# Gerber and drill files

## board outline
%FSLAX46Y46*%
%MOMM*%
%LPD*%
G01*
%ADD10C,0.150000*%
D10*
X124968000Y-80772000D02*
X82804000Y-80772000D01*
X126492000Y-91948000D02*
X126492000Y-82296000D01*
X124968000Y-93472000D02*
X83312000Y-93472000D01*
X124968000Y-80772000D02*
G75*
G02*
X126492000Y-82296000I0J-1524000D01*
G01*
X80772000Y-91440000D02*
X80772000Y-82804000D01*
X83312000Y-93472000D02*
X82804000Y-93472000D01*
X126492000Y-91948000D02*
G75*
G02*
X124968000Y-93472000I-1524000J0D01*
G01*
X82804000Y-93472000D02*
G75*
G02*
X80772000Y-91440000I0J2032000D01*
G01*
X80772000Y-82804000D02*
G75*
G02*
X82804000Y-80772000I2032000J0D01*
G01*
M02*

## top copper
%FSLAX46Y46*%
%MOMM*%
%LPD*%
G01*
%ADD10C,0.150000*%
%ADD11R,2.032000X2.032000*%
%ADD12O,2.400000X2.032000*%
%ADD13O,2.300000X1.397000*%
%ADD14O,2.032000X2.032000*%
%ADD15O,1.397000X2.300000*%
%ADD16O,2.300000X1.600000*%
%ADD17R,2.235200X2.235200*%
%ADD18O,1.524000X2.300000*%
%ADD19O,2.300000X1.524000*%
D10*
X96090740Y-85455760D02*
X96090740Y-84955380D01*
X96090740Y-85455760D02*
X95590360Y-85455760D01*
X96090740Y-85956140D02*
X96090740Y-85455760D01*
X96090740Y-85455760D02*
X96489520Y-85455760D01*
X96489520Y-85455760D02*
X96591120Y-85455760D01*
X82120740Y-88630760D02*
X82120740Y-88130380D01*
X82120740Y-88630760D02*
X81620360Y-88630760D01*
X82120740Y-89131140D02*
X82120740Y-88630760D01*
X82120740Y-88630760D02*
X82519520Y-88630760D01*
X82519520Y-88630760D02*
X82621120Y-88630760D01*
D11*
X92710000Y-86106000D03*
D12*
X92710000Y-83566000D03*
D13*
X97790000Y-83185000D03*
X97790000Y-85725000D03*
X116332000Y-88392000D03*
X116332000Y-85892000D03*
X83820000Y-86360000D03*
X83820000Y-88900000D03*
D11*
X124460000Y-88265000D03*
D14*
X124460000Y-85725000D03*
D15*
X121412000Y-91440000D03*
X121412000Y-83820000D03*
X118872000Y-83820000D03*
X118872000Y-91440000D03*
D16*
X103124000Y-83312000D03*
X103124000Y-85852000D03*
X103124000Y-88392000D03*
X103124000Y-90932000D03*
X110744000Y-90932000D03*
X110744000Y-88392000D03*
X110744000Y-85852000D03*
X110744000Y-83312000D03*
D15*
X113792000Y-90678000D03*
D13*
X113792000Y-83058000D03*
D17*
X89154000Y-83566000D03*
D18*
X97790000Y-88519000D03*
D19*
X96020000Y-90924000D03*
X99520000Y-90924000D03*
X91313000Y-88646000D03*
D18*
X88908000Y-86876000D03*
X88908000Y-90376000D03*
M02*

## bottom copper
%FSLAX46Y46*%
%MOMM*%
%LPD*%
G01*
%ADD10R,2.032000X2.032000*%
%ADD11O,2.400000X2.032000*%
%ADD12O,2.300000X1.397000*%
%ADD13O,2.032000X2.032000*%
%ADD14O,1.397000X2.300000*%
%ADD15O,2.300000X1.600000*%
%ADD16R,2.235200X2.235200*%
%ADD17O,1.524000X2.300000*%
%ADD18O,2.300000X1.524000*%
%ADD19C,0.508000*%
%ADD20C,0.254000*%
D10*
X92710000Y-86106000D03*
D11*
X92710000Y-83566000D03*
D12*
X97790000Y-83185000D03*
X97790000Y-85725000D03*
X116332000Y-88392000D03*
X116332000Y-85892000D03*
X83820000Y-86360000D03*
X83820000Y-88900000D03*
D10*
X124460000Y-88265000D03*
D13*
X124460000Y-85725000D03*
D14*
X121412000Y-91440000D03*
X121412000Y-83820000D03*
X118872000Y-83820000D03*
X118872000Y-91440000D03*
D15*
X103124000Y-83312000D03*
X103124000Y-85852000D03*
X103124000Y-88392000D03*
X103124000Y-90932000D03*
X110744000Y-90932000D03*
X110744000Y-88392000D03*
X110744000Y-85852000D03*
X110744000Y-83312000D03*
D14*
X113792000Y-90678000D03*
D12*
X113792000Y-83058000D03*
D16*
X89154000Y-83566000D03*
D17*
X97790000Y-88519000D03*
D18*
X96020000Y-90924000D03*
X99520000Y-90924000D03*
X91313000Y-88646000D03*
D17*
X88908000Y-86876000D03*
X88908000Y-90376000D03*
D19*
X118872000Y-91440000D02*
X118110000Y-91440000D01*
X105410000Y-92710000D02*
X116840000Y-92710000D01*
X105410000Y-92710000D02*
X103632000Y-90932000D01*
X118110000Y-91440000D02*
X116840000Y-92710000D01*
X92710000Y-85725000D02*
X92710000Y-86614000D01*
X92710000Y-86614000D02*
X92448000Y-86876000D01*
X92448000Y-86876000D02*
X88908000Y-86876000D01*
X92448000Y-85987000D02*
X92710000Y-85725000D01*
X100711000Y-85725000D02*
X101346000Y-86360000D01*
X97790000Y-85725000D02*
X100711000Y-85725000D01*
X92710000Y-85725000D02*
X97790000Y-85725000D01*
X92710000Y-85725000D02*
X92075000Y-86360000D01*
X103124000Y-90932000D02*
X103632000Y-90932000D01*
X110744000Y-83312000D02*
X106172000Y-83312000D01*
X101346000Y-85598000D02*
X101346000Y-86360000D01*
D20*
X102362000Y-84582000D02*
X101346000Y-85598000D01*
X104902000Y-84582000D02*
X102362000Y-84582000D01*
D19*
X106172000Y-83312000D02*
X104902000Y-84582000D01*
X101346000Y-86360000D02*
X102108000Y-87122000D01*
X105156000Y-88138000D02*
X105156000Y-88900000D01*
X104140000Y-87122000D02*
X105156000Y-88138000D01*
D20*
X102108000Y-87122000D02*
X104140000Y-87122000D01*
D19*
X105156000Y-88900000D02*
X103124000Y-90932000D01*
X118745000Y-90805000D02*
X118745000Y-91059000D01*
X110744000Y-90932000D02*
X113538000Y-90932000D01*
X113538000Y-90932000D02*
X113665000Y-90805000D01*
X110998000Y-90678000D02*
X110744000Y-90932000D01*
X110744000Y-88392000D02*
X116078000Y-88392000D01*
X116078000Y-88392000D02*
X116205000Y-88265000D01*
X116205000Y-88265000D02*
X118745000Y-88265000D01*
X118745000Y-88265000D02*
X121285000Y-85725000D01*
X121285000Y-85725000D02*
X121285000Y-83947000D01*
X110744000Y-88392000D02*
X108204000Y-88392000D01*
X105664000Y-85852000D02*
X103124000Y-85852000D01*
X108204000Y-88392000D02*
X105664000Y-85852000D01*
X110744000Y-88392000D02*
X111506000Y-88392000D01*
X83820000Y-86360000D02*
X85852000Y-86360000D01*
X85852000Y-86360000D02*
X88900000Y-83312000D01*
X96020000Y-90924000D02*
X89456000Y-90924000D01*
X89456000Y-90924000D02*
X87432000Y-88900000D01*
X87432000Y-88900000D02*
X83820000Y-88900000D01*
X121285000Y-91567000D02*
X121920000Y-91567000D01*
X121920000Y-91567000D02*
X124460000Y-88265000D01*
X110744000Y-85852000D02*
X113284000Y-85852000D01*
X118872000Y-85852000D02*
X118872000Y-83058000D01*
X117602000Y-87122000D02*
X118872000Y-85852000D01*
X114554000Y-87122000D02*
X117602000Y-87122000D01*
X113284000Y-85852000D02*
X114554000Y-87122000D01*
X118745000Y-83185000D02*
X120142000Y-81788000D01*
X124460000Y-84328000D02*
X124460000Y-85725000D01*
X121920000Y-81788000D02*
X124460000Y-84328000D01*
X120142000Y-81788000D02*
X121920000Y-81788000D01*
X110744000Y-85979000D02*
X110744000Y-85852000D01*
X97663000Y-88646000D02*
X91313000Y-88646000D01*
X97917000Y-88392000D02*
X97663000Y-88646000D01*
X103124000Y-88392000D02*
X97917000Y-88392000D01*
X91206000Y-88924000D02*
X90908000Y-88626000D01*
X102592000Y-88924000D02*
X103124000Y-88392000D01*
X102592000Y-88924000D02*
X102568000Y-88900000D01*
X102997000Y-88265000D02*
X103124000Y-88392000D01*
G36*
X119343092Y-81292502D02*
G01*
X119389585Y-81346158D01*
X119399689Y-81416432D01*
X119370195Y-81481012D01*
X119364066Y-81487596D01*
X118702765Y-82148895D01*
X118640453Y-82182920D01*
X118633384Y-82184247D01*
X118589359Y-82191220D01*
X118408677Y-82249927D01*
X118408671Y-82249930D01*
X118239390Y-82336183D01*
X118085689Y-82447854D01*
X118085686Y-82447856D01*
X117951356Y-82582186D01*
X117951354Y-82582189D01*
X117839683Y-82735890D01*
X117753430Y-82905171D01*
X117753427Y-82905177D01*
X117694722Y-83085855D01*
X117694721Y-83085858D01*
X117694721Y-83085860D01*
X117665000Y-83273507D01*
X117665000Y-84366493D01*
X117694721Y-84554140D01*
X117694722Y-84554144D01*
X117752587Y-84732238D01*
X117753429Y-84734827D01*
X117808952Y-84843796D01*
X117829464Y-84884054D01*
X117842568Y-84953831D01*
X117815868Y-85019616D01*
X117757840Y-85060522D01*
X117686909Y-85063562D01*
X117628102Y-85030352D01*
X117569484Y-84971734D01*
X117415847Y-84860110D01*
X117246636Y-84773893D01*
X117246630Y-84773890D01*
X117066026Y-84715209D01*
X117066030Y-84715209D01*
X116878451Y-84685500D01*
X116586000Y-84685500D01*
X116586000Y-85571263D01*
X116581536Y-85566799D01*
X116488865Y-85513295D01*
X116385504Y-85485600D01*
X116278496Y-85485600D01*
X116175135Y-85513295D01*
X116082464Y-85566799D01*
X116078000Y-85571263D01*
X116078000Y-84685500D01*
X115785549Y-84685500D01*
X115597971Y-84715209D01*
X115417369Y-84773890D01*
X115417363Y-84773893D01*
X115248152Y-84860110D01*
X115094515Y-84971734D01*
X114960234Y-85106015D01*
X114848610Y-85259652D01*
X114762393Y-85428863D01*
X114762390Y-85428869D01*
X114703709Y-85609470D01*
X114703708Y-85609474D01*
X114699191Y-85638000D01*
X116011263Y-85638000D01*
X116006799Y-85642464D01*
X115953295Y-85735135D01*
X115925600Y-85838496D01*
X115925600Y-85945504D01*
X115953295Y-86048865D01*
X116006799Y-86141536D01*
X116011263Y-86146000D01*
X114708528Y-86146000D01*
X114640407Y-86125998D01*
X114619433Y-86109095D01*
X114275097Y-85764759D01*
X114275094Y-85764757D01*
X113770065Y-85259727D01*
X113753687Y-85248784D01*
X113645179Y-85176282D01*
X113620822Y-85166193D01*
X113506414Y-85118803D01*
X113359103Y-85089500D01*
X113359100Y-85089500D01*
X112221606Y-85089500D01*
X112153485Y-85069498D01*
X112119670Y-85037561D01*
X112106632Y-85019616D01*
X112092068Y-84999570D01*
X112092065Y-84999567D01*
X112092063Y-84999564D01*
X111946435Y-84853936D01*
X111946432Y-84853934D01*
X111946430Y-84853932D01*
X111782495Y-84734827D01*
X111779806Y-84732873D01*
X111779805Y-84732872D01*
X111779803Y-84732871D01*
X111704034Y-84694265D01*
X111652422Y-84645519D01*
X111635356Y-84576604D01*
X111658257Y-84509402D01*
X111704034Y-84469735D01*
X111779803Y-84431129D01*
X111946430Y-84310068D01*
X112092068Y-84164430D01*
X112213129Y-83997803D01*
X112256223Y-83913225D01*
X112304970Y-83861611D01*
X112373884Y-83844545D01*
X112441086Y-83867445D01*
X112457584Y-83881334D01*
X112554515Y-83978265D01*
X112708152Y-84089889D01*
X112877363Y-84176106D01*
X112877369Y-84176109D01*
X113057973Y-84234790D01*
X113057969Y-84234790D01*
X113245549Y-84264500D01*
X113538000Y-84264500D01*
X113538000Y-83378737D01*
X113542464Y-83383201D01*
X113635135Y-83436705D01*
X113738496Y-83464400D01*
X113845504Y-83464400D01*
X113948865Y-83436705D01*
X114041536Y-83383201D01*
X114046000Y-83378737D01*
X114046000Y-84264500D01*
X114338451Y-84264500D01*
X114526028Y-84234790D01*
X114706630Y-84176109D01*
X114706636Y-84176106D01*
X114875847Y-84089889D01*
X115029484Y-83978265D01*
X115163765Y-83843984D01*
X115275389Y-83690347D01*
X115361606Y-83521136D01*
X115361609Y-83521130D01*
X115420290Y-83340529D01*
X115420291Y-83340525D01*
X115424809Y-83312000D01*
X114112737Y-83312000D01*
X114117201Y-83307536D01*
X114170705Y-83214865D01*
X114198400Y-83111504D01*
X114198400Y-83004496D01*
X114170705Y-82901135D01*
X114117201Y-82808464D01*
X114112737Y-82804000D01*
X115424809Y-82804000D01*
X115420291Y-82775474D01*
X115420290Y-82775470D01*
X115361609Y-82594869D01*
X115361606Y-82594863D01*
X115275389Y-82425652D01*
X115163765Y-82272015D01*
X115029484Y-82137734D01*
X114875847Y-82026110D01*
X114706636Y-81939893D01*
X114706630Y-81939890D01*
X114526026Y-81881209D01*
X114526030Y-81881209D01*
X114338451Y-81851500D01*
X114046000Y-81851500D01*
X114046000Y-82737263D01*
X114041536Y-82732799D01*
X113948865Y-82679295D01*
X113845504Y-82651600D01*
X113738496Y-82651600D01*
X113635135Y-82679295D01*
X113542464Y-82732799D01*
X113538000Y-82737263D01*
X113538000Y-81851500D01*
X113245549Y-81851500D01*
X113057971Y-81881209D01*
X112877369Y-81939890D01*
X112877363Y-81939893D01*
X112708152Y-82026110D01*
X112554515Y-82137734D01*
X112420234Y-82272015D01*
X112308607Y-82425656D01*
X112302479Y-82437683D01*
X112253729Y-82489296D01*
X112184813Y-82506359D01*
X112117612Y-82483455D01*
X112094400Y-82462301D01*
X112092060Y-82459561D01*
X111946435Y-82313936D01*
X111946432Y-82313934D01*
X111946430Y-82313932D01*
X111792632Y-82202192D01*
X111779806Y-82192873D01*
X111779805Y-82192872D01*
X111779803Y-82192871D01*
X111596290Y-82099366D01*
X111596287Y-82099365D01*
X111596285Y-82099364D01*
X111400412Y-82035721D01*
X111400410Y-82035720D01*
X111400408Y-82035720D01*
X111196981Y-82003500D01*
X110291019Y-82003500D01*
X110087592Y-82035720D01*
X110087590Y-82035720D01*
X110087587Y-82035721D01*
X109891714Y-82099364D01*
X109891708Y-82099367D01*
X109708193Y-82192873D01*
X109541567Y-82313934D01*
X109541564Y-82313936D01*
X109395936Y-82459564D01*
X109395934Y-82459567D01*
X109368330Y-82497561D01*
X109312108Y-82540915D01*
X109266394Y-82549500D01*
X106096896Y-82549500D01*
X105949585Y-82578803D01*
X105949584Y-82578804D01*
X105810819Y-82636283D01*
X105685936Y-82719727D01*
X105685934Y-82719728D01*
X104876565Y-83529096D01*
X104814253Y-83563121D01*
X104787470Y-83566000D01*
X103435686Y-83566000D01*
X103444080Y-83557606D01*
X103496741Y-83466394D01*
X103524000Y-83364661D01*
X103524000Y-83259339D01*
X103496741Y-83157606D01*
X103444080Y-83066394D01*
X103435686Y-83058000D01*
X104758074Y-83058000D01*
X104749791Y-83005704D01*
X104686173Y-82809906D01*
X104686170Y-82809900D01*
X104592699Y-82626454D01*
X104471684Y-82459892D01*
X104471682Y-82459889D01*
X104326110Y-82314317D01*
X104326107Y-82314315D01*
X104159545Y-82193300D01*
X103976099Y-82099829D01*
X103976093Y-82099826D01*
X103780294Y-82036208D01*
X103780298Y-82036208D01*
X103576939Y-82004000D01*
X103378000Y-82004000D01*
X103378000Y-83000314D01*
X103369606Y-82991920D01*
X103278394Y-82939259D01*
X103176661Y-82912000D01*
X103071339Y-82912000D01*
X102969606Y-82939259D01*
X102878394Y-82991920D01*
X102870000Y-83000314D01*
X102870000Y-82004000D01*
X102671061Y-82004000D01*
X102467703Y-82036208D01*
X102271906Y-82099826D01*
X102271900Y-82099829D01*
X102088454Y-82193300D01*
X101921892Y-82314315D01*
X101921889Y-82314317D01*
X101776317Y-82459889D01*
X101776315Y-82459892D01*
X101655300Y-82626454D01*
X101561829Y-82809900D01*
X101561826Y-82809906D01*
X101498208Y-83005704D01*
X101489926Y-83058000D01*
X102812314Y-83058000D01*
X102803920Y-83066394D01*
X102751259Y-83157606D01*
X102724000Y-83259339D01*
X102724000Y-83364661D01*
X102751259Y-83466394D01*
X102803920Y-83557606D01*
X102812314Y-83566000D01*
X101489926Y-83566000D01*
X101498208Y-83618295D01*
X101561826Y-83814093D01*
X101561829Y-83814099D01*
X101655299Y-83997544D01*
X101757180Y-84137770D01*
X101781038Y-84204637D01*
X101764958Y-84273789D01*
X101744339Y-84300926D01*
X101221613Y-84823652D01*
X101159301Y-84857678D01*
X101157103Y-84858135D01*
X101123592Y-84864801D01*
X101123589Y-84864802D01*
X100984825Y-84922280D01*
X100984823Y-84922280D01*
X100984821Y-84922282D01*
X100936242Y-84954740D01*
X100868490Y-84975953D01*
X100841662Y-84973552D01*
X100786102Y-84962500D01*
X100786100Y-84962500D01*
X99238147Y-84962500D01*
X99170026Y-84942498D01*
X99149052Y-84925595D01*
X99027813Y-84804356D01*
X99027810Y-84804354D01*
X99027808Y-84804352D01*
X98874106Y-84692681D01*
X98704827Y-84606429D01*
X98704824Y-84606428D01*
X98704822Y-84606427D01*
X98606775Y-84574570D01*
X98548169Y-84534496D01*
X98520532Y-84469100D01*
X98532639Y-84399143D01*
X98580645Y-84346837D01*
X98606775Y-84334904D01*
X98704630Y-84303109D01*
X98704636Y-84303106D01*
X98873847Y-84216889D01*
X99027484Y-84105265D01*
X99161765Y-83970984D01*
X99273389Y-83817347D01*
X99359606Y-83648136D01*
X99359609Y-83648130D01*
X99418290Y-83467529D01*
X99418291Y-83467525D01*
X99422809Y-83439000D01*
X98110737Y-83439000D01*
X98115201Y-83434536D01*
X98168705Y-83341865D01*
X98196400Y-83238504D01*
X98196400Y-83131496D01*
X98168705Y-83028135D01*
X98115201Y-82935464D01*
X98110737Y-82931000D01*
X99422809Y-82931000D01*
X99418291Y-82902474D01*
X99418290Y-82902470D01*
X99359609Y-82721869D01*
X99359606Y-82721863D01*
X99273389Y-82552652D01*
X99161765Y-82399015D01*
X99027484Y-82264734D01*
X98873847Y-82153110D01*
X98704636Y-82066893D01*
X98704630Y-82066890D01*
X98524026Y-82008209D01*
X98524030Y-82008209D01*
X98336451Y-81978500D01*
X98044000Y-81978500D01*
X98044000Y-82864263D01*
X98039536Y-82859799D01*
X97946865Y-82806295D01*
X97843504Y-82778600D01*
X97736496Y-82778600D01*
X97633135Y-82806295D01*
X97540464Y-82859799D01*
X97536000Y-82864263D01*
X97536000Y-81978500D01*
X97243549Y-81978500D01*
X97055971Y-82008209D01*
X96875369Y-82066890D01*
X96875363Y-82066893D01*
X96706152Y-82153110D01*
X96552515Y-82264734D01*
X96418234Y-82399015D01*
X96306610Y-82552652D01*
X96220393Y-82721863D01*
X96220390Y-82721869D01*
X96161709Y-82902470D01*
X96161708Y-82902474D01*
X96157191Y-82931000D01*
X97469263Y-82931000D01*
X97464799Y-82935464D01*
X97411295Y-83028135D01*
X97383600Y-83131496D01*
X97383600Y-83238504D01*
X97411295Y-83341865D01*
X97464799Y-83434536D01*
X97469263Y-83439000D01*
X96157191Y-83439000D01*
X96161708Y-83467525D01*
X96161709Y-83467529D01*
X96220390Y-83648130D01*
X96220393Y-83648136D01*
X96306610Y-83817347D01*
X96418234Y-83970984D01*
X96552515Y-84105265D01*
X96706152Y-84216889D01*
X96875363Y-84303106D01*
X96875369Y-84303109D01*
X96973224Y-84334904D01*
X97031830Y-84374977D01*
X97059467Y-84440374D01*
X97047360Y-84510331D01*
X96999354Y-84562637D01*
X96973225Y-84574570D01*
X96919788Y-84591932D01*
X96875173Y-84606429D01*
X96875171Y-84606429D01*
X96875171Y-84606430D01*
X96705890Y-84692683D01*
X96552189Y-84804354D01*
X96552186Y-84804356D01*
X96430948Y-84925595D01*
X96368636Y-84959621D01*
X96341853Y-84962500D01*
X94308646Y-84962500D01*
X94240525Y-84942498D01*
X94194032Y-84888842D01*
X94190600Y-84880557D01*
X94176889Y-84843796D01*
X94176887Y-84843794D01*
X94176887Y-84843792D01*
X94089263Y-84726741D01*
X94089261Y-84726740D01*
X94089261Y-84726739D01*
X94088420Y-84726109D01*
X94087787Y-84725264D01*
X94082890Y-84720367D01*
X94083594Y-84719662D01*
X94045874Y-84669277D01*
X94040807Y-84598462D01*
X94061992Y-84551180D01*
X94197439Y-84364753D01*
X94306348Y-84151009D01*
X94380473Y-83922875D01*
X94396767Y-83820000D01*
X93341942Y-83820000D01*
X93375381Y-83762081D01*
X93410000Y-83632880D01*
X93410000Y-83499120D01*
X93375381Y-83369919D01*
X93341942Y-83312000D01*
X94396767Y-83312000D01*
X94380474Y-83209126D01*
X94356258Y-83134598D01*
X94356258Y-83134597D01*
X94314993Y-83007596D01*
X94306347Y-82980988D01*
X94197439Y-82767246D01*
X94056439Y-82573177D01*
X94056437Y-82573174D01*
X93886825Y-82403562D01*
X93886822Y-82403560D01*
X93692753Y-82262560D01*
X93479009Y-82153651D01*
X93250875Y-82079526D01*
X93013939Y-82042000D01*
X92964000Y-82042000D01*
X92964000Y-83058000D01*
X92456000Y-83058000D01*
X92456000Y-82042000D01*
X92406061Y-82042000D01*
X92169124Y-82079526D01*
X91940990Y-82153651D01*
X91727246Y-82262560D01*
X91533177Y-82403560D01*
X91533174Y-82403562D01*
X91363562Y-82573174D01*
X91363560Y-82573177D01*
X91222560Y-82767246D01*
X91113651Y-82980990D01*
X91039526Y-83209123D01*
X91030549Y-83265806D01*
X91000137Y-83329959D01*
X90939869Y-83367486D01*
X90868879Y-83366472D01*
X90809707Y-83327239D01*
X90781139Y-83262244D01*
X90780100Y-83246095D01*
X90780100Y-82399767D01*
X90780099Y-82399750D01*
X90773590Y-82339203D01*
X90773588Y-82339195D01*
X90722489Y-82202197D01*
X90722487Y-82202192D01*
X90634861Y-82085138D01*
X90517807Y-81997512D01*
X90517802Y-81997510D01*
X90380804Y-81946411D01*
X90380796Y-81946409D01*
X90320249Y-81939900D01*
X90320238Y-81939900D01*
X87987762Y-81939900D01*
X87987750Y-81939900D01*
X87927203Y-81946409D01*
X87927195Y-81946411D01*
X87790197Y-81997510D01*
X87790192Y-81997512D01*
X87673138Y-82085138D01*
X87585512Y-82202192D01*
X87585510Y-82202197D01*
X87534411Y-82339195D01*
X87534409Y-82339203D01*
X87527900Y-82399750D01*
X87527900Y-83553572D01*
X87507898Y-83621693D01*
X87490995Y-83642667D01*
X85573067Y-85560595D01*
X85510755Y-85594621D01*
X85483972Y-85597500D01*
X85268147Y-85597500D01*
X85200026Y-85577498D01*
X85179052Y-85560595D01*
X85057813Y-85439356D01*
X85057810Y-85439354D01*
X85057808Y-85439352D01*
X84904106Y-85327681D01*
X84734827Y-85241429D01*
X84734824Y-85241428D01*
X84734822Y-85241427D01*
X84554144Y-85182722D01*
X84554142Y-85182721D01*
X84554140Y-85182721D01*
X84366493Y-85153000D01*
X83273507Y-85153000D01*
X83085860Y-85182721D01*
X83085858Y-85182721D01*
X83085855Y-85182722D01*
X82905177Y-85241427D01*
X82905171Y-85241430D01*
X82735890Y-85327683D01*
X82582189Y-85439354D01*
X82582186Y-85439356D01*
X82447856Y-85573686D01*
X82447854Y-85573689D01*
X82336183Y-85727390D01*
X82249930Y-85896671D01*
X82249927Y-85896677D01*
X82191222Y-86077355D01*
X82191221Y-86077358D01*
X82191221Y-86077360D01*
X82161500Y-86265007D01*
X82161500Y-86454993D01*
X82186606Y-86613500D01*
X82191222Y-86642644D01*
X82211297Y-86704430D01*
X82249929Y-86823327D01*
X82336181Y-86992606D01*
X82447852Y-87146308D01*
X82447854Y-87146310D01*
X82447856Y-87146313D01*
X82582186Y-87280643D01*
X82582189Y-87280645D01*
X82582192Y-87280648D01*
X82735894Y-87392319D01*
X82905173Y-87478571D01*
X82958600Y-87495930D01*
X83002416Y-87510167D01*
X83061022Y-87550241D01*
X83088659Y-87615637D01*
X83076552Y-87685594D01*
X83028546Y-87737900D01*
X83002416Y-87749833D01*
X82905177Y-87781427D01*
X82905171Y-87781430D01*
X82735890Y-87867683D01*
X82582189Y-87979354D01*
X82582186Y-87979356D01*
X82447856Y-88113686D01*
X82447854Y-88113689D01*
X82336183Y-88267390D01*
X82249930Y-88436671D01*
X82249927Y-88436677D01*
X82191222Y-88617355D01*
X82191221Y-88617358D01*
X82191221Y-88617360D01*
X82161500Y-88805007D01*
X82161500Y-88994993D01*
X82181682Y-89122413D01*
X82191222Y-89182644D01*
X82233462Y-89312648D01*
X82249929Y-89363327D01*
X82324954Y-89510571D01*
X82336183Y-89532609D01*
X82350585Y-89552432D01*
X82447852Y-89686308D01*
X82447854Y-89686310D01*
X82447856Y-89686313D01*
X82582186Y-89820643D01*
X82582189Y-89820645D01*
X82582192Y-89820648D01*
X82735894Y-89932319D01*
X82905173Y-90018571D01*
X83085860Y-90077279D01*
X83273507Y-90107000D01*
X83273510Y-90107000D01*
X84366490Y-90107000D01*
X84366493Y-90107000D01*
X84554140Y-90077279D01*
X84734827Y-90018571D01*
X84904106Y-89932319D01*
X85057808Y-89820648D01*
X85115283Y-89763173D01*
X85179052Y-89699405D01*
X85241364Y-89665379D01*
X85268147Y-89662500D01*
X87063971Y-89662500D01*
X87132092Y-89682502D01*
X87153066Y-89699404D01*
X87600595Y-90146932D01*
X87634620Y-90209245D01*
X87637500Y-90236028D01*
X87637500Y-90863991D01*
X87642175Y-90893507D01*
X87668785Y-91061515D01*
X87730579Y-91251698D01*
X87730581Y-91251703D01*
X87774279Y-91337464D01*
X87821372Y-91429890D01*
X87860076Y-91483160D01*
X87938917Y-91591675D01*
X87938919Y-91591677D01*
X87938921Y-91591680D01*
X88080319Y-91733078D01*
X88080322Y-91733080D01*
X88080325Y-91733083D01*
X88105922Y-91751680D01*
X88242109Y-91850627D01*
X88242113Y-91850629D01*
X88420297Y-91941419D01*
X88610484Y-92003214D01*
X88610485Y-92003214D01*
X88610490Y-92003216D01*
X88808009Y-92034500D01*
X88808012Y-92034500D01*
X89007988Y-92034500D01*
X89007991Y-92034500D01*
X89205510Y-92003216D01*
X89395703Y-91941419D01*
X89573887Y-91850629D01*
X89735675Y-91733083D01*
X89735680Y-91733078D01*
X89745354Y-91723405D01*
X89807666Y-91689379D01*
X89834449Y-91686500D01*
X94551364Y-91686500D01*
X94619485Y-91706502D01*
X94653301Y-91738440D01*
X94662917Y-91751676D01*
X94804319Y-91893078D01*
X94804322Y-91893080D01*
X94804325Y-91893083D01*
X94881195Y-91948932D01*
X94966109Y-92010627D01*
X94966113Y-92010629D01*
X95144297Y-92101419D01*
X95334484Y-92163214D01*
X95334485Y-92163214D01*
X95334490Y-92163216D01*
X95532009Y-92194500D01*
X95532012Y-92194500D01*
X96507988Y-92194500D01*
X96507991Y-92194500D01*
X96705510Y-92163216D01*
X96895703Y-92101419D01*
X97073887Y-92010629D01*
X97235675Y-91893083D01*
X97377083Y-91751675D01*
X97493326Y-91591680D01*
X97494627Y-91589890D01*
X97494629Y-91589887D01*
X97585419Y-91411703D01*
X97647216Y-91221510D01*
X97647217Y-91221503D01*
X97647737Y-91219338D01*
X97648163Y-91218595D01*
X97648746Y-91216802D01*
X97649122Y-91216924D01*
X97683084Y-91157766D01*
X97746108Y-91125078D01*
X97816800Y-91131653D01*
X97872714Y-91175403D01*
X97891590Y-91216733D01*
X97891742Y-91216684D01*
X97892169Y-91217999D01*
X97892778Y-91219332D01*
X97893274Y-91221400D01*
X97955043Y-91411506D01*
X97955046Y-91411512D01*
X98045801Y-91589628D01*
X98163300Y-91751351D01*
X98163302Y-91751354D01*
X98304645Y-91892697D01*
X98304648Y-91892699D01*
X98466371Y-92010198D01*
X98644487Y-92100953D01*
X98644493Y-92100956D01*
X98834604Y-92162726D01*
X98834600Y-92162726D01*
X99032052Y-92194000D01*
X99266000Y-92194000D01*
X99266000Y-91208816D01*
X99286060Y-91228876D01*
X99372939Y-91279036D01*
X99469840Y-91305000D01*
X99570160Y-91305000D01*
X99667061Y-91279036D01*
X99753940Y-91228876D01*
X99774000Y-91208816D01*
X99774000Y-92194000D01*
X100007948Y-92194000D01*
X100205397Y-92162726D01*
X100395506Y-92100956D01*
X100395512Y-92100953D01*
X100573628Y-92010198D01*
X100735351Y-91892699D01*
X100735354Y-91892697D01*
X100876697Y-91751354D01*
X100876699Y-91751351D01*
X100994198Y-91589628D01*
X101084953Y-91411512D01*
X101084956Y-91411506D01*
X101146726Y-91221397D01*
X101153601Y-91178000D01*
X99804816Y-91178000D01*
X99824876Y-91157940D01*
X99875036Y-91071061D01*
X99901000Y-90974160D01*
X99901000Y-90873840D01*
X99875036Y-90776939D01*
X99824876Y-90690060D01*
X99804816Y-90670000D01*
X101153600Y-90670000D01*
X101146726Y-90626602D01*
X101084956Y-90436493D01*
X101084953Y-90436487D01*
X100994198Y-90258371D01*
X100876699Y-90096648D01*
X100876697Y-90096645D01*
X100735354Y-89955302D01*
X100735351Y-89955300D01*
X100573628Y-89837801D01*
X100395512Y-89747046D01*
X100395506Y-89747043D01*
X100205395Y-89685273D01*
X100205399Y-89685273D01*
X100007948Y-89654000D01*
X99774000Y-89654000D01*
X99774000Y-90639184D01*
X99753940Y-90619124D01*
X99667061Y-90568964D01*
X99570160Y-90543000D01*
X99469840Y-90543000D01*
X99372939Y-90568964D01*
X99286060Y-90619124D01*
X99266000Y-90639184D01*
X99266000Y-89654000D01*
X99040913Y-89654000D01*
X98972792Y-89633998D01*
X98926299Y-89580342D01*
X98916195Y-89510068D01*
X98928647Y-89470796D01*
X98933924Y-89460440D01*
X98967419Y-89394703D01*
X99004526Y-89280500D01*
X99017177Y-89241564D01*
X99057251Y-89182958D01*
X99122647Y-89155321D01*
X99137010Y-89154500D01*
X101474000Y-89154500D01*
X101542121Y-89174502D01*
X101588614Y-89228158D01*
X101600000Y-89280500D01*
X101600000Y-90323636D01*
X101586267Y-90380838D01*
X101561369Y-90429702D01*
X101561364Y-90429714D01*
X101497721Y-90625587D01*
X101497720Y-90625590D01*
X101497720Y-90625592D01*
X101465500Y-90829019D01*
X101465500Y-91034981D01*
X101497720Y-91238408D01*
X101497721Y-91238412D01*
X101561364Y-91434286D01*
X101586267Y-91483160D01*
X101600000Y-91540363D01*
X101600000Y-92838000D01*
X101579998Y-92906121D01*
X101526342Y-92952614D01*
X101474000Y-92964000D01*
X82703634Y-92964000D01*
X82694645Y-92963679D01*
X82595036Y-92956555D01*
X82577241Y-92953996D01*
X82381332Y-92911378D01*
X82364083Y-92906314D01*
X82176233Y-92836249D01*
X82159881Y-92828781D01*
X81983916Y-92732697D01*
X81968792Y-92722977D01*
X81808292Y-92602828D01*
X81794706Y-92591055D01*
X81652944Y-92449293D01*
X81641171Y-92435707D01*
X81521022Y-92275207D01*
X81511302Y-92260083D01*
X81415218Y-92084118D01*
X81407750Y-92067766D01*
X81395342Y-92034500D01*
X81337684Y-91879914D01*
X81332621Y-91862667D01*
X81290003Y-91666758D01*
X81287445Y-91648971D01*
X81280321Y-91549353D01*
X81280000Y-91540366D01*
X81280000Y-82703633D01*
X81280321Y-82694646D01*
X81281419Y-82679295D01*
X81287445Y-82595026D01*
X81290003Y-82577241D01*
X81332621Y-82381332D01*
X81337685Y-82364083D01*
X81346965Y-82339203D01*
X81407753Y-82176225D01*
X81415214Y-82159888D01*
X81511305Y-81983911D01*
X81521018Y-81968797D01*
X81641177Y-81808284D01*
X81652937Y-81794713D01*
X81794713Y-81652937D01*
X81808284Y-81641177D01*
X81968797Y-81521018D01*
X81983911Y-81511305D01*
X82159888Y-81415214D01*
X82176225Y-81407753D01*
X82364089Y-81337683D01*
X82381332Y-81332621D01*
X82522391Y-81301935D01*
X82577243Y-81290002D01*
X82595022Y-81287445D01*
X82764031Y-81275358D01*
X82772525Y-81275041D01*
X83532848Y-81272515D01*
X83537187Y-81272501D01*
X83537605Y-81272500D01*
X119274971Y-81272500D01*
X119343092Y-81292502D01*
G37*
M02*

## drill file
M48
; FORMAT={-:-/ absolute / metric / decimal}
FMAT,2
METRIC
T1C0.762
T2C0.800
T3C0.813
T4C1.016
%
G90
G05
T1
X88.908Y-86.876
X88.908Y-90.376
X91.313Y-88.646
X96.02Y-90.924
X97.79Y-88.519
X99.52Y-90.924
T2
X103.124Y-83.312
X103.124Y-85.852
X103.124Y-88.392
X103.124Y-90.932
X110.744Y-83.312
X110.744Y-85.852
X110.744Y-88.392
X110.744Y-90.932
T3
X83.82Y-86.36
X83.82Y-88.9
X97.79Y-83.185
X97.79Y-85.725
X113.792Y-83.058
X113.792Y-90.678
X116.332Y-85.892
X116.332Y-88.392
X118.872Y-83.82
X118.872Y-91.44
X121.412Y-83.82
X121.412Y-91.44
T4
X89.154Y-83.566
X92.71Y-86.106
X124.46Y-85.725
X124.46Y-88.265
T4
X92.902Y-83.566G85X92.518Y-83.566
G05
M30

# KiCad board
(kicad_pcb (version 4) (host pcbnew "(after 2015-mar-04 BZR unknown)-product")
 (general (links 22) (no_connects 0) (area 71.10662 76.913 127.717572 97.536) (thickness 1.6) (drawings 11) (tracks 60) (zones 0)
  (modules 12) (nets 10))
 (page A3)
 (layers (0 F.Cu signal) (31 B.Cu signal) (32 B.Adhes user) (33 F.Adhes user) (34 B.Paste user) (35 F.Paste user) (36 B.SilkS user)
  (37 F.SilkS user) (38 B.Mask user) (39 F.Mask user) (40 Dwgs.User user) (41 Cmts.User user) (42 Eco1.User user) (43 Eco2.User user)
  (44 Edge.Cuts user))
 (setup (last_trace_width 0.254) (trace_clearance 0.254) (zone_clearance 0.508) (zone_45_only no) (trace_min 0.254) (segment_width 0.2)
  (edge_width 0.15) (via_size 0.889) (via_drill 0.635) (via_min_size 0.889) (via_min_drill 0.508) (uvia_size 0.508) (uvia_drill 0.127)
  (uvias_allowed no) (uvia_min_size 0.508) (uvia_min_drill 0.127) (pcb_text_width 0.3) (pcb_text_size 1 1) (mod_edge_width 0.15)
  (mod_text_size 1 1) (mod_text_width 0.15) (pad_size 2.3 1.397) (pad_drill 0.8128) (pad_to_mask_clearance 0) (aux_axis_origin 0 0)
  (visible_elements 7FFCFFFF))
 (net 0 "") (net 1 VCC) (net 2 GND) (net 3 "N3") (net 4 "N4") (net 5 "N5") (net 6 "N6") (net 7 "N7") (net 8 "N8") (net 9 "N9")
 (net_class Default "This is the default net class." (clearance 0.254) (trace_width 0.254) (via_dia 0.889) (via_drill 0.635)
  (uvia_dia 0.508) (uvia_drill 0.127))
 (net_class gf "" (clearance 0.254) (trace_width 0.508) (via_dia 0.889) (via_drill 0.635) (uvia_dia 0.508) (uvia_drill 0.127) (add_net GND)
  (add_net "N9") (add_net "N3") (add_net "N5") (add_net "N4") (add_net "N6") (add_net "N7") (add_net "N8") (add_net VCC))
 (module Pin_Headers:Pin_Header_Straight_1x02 (layer F.Cu) (at 92.71 86.106 180)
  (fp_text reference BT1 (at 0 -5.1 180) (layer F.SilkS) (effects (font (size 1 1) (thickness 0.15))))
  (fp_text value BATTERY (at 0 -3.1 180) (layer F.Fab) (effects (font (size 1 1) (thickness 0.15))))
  (pad 1 thru_hole rect (at 0 0 180) (size 2.032 2.032) (drill 1.016) (layers *.Cu *.Mask F.SilkS) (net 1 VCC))
  (pad 2 thru_hole oval (at 0 2.54 180) (size 2.4 2.032) (drill oval 1.4 1.016) (layers *.Cu *.Mask F.SilkS) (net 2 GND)))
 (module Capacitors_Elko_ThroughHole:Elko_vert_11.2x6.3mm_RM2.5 (layer F.Cu) (at 97.79 85.725 90)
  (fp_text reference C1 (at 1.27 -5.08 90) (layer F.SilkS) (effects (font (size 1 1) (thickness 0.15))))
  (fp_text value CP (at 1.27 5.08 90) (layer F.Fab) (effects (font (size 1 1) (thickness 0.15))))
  (fp_line (start 0.26924 -1.69926) (end 0.76962 -1.69926) (layer F.Cu) (width 0.15))
  (fp_line (start 0.26924 -1.69926) (end 0.26924 -2.19964) (layer F.Cu) (width 0.15))
  (fp_line (start -0.23114 -1.69926) (end 0.26924 -1.69926) (layer F.Cu) (width 0.15))
  (fp_line (start 0.26924 -1.69926) (end 0.26924 -1.30048) (layer F.Cu) (width 0.15))
  (fp_line (start 0.26924 -1.30048) (end 0.26924 -1.19888) (layer F.Cu) (width 0.15))
  (pad 2 thru_hole oval (at 2.54 0 90) (size 1.397 2.3) (drill 0.8128) (layers *.Cu *.Mask F.SilkS) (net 2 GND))
  (pad 1 thru_hole oval (at 0 0 90) (size 1.397 2.3) (drill 0.8128) (layers *.Cu *.Mask F.SilkS) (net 1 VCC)))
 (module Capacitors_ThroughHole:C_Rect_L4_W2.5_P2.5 (layer F.Cu) (at 116.332 88.392 90)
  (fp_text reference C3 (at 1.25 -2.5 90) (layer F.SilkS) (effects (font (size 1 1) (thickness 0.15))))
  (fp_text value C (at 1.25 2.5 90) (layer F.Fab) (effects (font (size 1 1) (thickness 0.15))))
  (pad 1 thru_hole oval (at 0 0 90) (size 1.397 2.3) (drill 0.8128) (layers *.Cu *.Mask F.SilkS) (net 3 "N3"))
  (pad 2 thru_hole oval (at 2.5 0 90) (size 1.397 2.3) (drill 0.8128) (layers *.Cu *.Mask F.SilkS) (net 2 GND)))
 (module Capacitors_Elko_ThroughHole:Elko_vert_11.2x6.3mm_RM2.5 (layer F.Cu) (at 83.82 88.9 90)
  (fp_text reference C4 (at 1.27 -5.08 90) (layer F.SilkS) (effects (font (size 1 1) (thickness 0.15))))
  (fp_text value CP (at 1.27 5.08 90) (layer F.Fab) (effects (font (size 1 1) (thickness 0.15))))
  (fp_line (start 0.26924 -1.69926) (end 0.76962 -1.69926) (layer F.Cu) (width 0.15))
  (fp_line (start 0.26924 -1.69926) (end 0.26924 -2.19964) (layer F.Cu) (width 0.15))
  (fp_line (start -0.23114 -1.69926) (end 0.26924 -1.69926) (layer F.Cu) (width 0.15))
  (fp_line (start 0.26924 -1.69926) (end 0.26924 -1.30048) (layer F.Cu) (width 0.15))
  (fp_line (start 0.26924 -1.30048) (end 0.26924 -1.19888) (layer F.Cu) (width 0.15))
  (pad 2 thru_hole oval (at 2.54 0 90) (size 1.397 2.3) (drill 0.8128) (layers *.Cu *.Mask F.SilkS) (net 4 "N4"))
  (pad 1 thru_hole oval (at 0 0 90) (size 1.397 2.3) (drill 0.8128) (layers *.Cu *.Mask F.SilkS) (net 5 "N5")))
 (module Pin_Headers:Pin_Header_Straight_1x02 (layer F.Cu) (at 124.46 88.265 180)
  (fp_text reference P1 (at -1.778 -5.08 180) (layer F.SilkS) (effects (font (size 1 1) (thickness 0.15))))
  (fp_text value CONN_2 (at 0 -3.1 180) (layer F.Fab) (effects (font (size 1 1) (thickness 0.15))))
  (pad 1 thru_hole rect (at 0 0 180) (size 2.032 2.032) (drill 1.016) (layers *.Cu *.Mask F.SilkS) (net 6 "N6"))
  (pad 2 thru_hole oval (at 0 2.54 180) (size 2.032 2.032) (drill 1.016) (layers *.Cu *.Mask F.SilkS) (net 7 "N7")))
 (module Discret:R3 (layer F.Cu) (at 121.412 87.63 90)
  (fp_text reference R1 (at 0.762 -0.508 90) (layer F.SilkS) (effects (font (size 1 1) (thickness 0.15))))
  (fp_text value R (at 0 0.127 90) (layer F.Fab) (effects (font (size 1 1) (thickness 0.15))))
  (pad 1 thru_hole oval (at -3.81 0 90) (size 2.3 1.397) (drill 0.8128) (layers *.Cu *.Mask F.SilkS) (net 6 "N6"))
  (pad 2 thru_hole oval (at 3.81 0 90) (size 2.3 1.397) (drill 0.8128) (layers *.Cu *.Mask F.SilkS) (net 3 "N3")))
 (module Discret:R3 (layer F.Cu) (at 118.872 87.63 270)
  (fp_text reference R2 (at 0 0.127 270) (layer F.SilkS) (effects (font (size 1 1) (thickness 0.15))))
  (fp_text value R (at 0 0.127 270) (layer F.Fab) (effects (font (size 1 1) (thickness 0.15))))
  (pad 1 thru_hole oval (at -3.81 0 270) (size 2.3 1.397) (drill 0.8128) (layers *.Cu *.Mask F.SilkS) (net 7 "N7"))
  (pad 2 thru_hole oval (at 3.81 0 270) (size 2.3 1.397) (drill 0.8128) (layers *.Cu *.Mask F.SilkS) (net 1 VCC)))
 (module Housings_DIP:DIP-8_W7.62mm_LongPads (layer F.Cu) (at 103.124 83.312)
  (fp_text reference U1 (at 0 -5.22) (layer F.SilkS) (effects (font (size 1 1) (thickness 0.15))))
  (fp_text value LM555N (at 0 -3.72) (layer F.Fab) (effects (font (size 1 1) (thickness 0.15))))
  (pad 1 thru_hole oval (at 0 0) (size 2.3 1.6) (drill 0.8) (layers *.Cu *.Mask F.SilkS) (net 2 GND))
  (pad 2 thru_hole oval (at 0 2.54) (size 2.3 1.6) (drill 0.8) (layers *.Cu *.Mask F.SilkS) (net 3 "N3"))
  (pad 3 thru_hole oval (at 0 5.08) (size 2.3 1.6) (drill 0.8) (layers *.Cu *.Mask F.SilkS) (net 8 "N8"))
  (pad 4 thru_hole oval (at 0 7.62) (size 2.3 1.6) (drill 0.8) (layers *.Cu *.Mask F.SilkS) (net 1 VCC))
  (pad 5 thru_hole oval (at 7.62 7.62) (size 2.3 1.6) (drill 0.8) (layers *.Cu *.Mask F.SilkS) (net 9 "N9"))
  (pad 6 thru_hole oval (at 7.62 5.08) (size 2.3 1.6) (drill 0.8) (layers *.Cu *.Mask F.SilkS) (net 3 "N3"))
  (pad 7 thru_hole oval (at 7.62 2.54) (size 2.3 1.6) (drill 0.8) (layers *.Cu *.Mask F.SilkS) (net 7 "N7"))
  (pad 8 thru_hole oval (at 7.62 0) (size 2.3 1.6) (drill 0.8) (layers *.Cu *.Mask F.SilkS) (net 1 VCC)))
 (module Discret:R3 (layer F.Cu) (at 113.792 86.868 90)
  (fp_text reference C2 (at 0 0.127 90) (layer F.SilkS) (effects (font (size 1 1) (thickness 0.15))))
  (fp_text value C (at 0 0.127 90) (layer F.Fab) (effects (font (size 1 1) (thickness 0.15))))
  (pad 1 thru_hole oval (at -3.81 0 90) (size 2.3 1.397) (drill 0.8128) (layers *.Cu *.Mask F.SilkS) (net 9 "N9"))
  (pad 2 thru_hole oval (at 3.81 0 180) (size 2.3 1.397) (drill 0.8128) (layers *.Cu *.Mask F.SilkS) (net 2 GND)))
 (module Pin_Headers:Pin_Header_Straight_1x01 (layer F.Cu) (at 89.154 83.566 180)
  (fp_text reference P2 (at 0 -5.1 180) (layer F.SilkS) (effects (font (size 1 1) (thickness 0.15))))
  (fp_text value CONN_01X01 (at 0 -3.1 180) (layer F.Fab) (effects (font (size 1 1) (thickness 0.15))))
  (pad 1 thru_hole rect (at 0 0 180) (size 2.2352 2.2352) (drill 1.016) (layers *.Cu *.Mask F.SilkS) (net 4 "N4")))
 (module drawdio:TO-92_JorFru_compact (layer F.Cu) (at 96.52 90.424)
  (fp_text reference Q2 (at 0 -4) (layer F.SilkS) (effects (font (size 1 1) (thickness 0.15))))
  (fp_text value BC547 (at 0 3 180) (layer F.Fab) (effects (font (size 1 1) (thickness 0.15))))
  (pad 2 thru_hole oval (at 1.27 -1.905 90) (size 2.3 1.524) (drill 0.762) (layers *.Cu *.Mask F.SilkS) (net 8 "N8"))
  (pad 1 thru_hole oval (at -0.5 0.5) (size 2.3 1.524) (drill 0.762) (layers *.Cu *.Mask F.SilkS) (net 5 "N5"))
  (pad 3 thru_hole oval (at 3 0.5) (size 2.3 1.524) (drill 0.762) (layers *.Cu *.Mask F.SilkS) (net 2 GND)))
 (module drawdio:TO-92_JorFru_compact (layer F.Cu) (at 89.408 87.376 270)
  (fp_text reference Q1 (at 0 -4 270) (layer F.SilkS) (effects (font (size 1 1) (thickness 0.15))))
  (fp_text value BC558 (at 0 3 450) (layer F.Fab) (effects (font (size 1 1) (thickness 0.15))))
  (pad 2 thru_hole oval (at 1.27 -1.905) (size 2.3 1.524) (drill 0.762) (layers *.Cu *.Mask F.SilkS) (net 8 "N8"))
  (pad 1 thru_hole oval (at -0.5 0.5 270) (size 2.3 1.524) (drill 0.762) (layers *.Cu *.Mask F.SilkS) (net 1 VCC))
  (pad 3 thru_hole oval (at 3 0.5 270) (size 2.3 1.524) (drill 0.762) (layers *.Cu *.Mask F.SilkS) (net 5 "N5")))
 (gr_line (start 124.968 80.772) (end 82.804 80.772) (angle 90) (layer Edge.Cuts) (width 0.15))
 (gr_line (start 126.492 91.948) (end 126.492 82.296) (angle 90) (layer Edge.Cuts) (width 0.15))
 (gr_line (start 124.968 93.472) (end 83.312 93.472) (angle 90) (layer Edge.Cuts) (width 0.15))
 (gr_arc (start 124.968 82.296) (end 124.968 80.772) (angle 90) (layer Edge.Cuts) (width 0.15))
 (gr_line (start 80.772 91.44) (end 80.772 82.804) (angle 90) (layer Edge.Cuts) (width 0.15))
 (gr_line (start 83.312 93.472) (end 82.804 93.472) (angle 90) (layer Edge.Cuts) (width 0.15))
 (gr_arc (start 124.968 91.948) (end 126.492 91.948) (angle 90) (layer Edge.Cuts) (width 0.15))
 (gr_arc (start 82.804 91.44) (end 82.804 93.472) (angle 90) (layer Edge.Cuts) (width 0.15))
 (gr_arc (start 82.804 82.804) (end 80.772 82.804) (angle 90) (layer Edge.Cuts) (width 0.15))
 (segment (start 118.872 91.44) (end 118.11 91.44) (width 0.508) (layer B.Cu) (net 1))
 (segment (start 105.41 92.71) (end 116.84 92.71) (width 0.508) (layer B.Cu) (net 1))
 (segment (start 105.41 92.71) (end 103.632 90.932) (width 0.508) (layer B.Cu) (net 1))
 (segment (start 118.11 91.44) (end 116.84 92.71) (width 0.508) (layer B.Cu) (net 1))
 (segment (start 92.71 85.725) (end 92.71 86.614) (width 0.508) (layer B.Cu) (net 1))
 (segment (start 92.71 86.614) (end 92.448 86.876) (width 0.508) (layer B.Cu) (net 1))
 (segment (start 92.448 86.876) (end 88.908 86.876) (width 0.508) (layer B.Cu) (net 1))
 (segment (start 92.448 85.987) (end 92.71 85.725) (width 0.508) (layer B.Cu) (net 1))
 (segment (start 100.711 85.725) (end 101.346 86.36) (width 0.508) (layer B.Cu) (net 1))
 (segment (start 97.79 85.725) (end 100.711 85.725) (width 0.508) (layer B.Cu) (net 1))
 (segment (start 92.71 85.725) (end 97.79 85.725) (width 0.508) (layer B.Cu) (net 1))
 (segment (start 92.71 85.725) (end 92.075 86.36) (width 0.508) (layer B.Cu) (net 1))
 (segment (start 103.124 90.932) (end 103.632 90.932) (width 0.508) (layer B.Cu) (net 1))
 (segment (start 110.744 83.312) (end 106.172 83.312) (width 0.508) (layer B.Cu) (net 1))
 (segment (start 101.346 85.598) (end 101.346 86.36) (width 0.508) (layer B.Cu) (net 1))
 (segment (start 102.362 84.582) (end 101.346 85.598) (width 0.254) (layer B.Cu) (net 1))
 (segment (start 104.902 84.582) (end 102.362 84.582) (width 0.254) (layer B.Cu) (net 1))
 (segment (start 106.172 83.312) (end 104.902 84.582) (width 0.508) (layer B.Cu) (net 1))
 (segment (start 101.346 86.36) (end 102.108 87.122) (width 0.508) (layer B.Cu) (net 1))
 (segment (start 105.156 88.138) (end 105.156 88.9) (width 0.508) (layer B.Cu) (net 1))
 (segment (start 104.14 87.122) (end 105.156 88.138) (width 0.508) (layer B.Cu) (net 1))
 (segment (start 102.108 87.122) (end 104.14 87.122) (width 0.254) (layer B.Cu) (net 1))
 (segment (start 105.156 88.9) (end 103.124 90.932) (width 0.508) (layer B.Cu) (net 1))
 (segment (start 118.745 90.805) (end 118.745 91.059) (width 0.508) (layer B.Cu) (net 1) (status 30))
 (segment (start 110.744 90.932) (end 113.538 90.932) (width 0.508) (layer B.Cu) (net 9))
 (segment (start 113.538 90.932) (end 113.665 90.805) (width 0.508) (layer B.Cu) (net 9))
 (segment (start 110.998 90.678) (end 110.744 90.932) (width 0.508) (layer B.Cu) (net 9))
 (segment (start 110.744 88.392) (end 116.078 88.392) (width 0.508) (layer B.Cu) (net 3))
 (segment (start 116.078 88.392) (end 116.205 88.265) (width 0.508) (layer B.Cu) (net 3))
 (segment (start 116.205 88.265) (end 118.745 88.265) (width 0.508) (layer B.Cu) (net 3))
 (segment (start 118.745 88.265) (end 121.285 85.725) (width 0.508) (layer B.Cu) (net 3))
 (segment (start 121.285 85.725) (end 121.285 83.947) (width 0.508) (layer B.Cu) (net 3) (status 20))
 (segment (start 110.744 88.392) (end 108.204 88.392) (width 0.508) (layer B.Cu) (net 3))
 (segment (start 105.664 85.852) (end 103.124 85.852) (width 0.508) (layer B.Cu) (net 3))
 (segment (start 108.204 88.392) (end 105.664 85.852) (width 0.508) (layer B.Cu) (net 3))
 (segment (start 110.744 88.392) (end 111.506 88.392) (width 0.508) (layer B.Cu) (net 3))
 (segment (start 83.82 86.36) (end 85.852 86.36) (width 0.508) (layer B.Cu) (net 4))
 (segment (start 85.852 86.36) (end 88.9 83.312) (width 0.508) (layer B.Cu) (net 4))
 (segment (start 96.02 90.924) (end 89.456 90.924) (width 0.508) (layer B.Cu) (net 5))
 (segment (start 89.456 90.924) (end 87.432 88.9) (width 0.508) (layer B.Cu) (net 5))
 (segment (start 87.432 88.9) (end 83.82 88.9) (width 0.508) (layer B.Cu) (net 5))
 (segment (start 121.285 91.567) (end 121.92 91.567) (width 0.508) (layer B.Cu) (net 6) (status 30))
 (segment (start 121.92 91.567) (end 124.46 88.265) (width 0.508) (layer B.Cu) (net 6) (status 10))
 (segment (start 110.744 85.852) (end 113.284 85.852) (width 0.508) (layer B.Cu) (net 7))
 (segment (start 118.872 85.852) (end 118.872 83.058) (width 0.508) (layer B.Cu) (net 7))
 (segment (start 117.602 87.122) (end 118.872 85.852) (width 0.508) (layer B.Cu) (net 7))
 (segment (start 114.554 87.122) (end 117.602 87.122) (width 0.508) (layer B.Cu) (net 7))
 (segment (start 113.284 85.852) (end 114.554 87.122) (width 0.508) (layer B.Cu) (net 7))
 (segment (start 118.745 83.185) (end 120.142 81.788) (width 0.508) (layer B.Cu) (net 7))
 (segment (start 124.46 84.328) (end 124.46 85.725) (width 0.508) (layer B.Cu) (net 7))
 (segment (start 121.92 81.788) (end 124.46 84.328) (width 0.508) (layer B.Cu) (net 7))
 (segment (start 120.142 81.788) (end 121.92 81.788) (width 0.508) (layer B.Cu) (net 7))
 (segment (start 110.744 85.979) (end 110.744 85.852) (width 0.508) (layer B.Cu) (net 7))
 (segment (start 97.663 88.646) (end 91.313 88.646) (width 0.508) (layer B.Cu) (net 8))
 (segment (start 97.917 88.392) (end 97.663 88.646) (width 0.508) (layer B.Cu) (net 8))
 (segment (start 103.124 88.392) (end 97.917 88.392) (width 0.508) (layer B.Cu) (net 8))
 (segment (start 91.206 88.924) (end 90.908 88.626) (width 0.508) (layer B.Cu) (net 8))
 (segment (start 102.592 88.924) (end 103.124 88.392) (width 0.508) (layer B.Cu) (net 8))
 (segment (start 102.592 88.924) (end 102.568 88.9) (width 0.508) (layer B.Cu) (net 8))
 (segment (start 102.997 88.265) (end 103.124 88.392) (width 0.508) (layer B.Cu) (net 8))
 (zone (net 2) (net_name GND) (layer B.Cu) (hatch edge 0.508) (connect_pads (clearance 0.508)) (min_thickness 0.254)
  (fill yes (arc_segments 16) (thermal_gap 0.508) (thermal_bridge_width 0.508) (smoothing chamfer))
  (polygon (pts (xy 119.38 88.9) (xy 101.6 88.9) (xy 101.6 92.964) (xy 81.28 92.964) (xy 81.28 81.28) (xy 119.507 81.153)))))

